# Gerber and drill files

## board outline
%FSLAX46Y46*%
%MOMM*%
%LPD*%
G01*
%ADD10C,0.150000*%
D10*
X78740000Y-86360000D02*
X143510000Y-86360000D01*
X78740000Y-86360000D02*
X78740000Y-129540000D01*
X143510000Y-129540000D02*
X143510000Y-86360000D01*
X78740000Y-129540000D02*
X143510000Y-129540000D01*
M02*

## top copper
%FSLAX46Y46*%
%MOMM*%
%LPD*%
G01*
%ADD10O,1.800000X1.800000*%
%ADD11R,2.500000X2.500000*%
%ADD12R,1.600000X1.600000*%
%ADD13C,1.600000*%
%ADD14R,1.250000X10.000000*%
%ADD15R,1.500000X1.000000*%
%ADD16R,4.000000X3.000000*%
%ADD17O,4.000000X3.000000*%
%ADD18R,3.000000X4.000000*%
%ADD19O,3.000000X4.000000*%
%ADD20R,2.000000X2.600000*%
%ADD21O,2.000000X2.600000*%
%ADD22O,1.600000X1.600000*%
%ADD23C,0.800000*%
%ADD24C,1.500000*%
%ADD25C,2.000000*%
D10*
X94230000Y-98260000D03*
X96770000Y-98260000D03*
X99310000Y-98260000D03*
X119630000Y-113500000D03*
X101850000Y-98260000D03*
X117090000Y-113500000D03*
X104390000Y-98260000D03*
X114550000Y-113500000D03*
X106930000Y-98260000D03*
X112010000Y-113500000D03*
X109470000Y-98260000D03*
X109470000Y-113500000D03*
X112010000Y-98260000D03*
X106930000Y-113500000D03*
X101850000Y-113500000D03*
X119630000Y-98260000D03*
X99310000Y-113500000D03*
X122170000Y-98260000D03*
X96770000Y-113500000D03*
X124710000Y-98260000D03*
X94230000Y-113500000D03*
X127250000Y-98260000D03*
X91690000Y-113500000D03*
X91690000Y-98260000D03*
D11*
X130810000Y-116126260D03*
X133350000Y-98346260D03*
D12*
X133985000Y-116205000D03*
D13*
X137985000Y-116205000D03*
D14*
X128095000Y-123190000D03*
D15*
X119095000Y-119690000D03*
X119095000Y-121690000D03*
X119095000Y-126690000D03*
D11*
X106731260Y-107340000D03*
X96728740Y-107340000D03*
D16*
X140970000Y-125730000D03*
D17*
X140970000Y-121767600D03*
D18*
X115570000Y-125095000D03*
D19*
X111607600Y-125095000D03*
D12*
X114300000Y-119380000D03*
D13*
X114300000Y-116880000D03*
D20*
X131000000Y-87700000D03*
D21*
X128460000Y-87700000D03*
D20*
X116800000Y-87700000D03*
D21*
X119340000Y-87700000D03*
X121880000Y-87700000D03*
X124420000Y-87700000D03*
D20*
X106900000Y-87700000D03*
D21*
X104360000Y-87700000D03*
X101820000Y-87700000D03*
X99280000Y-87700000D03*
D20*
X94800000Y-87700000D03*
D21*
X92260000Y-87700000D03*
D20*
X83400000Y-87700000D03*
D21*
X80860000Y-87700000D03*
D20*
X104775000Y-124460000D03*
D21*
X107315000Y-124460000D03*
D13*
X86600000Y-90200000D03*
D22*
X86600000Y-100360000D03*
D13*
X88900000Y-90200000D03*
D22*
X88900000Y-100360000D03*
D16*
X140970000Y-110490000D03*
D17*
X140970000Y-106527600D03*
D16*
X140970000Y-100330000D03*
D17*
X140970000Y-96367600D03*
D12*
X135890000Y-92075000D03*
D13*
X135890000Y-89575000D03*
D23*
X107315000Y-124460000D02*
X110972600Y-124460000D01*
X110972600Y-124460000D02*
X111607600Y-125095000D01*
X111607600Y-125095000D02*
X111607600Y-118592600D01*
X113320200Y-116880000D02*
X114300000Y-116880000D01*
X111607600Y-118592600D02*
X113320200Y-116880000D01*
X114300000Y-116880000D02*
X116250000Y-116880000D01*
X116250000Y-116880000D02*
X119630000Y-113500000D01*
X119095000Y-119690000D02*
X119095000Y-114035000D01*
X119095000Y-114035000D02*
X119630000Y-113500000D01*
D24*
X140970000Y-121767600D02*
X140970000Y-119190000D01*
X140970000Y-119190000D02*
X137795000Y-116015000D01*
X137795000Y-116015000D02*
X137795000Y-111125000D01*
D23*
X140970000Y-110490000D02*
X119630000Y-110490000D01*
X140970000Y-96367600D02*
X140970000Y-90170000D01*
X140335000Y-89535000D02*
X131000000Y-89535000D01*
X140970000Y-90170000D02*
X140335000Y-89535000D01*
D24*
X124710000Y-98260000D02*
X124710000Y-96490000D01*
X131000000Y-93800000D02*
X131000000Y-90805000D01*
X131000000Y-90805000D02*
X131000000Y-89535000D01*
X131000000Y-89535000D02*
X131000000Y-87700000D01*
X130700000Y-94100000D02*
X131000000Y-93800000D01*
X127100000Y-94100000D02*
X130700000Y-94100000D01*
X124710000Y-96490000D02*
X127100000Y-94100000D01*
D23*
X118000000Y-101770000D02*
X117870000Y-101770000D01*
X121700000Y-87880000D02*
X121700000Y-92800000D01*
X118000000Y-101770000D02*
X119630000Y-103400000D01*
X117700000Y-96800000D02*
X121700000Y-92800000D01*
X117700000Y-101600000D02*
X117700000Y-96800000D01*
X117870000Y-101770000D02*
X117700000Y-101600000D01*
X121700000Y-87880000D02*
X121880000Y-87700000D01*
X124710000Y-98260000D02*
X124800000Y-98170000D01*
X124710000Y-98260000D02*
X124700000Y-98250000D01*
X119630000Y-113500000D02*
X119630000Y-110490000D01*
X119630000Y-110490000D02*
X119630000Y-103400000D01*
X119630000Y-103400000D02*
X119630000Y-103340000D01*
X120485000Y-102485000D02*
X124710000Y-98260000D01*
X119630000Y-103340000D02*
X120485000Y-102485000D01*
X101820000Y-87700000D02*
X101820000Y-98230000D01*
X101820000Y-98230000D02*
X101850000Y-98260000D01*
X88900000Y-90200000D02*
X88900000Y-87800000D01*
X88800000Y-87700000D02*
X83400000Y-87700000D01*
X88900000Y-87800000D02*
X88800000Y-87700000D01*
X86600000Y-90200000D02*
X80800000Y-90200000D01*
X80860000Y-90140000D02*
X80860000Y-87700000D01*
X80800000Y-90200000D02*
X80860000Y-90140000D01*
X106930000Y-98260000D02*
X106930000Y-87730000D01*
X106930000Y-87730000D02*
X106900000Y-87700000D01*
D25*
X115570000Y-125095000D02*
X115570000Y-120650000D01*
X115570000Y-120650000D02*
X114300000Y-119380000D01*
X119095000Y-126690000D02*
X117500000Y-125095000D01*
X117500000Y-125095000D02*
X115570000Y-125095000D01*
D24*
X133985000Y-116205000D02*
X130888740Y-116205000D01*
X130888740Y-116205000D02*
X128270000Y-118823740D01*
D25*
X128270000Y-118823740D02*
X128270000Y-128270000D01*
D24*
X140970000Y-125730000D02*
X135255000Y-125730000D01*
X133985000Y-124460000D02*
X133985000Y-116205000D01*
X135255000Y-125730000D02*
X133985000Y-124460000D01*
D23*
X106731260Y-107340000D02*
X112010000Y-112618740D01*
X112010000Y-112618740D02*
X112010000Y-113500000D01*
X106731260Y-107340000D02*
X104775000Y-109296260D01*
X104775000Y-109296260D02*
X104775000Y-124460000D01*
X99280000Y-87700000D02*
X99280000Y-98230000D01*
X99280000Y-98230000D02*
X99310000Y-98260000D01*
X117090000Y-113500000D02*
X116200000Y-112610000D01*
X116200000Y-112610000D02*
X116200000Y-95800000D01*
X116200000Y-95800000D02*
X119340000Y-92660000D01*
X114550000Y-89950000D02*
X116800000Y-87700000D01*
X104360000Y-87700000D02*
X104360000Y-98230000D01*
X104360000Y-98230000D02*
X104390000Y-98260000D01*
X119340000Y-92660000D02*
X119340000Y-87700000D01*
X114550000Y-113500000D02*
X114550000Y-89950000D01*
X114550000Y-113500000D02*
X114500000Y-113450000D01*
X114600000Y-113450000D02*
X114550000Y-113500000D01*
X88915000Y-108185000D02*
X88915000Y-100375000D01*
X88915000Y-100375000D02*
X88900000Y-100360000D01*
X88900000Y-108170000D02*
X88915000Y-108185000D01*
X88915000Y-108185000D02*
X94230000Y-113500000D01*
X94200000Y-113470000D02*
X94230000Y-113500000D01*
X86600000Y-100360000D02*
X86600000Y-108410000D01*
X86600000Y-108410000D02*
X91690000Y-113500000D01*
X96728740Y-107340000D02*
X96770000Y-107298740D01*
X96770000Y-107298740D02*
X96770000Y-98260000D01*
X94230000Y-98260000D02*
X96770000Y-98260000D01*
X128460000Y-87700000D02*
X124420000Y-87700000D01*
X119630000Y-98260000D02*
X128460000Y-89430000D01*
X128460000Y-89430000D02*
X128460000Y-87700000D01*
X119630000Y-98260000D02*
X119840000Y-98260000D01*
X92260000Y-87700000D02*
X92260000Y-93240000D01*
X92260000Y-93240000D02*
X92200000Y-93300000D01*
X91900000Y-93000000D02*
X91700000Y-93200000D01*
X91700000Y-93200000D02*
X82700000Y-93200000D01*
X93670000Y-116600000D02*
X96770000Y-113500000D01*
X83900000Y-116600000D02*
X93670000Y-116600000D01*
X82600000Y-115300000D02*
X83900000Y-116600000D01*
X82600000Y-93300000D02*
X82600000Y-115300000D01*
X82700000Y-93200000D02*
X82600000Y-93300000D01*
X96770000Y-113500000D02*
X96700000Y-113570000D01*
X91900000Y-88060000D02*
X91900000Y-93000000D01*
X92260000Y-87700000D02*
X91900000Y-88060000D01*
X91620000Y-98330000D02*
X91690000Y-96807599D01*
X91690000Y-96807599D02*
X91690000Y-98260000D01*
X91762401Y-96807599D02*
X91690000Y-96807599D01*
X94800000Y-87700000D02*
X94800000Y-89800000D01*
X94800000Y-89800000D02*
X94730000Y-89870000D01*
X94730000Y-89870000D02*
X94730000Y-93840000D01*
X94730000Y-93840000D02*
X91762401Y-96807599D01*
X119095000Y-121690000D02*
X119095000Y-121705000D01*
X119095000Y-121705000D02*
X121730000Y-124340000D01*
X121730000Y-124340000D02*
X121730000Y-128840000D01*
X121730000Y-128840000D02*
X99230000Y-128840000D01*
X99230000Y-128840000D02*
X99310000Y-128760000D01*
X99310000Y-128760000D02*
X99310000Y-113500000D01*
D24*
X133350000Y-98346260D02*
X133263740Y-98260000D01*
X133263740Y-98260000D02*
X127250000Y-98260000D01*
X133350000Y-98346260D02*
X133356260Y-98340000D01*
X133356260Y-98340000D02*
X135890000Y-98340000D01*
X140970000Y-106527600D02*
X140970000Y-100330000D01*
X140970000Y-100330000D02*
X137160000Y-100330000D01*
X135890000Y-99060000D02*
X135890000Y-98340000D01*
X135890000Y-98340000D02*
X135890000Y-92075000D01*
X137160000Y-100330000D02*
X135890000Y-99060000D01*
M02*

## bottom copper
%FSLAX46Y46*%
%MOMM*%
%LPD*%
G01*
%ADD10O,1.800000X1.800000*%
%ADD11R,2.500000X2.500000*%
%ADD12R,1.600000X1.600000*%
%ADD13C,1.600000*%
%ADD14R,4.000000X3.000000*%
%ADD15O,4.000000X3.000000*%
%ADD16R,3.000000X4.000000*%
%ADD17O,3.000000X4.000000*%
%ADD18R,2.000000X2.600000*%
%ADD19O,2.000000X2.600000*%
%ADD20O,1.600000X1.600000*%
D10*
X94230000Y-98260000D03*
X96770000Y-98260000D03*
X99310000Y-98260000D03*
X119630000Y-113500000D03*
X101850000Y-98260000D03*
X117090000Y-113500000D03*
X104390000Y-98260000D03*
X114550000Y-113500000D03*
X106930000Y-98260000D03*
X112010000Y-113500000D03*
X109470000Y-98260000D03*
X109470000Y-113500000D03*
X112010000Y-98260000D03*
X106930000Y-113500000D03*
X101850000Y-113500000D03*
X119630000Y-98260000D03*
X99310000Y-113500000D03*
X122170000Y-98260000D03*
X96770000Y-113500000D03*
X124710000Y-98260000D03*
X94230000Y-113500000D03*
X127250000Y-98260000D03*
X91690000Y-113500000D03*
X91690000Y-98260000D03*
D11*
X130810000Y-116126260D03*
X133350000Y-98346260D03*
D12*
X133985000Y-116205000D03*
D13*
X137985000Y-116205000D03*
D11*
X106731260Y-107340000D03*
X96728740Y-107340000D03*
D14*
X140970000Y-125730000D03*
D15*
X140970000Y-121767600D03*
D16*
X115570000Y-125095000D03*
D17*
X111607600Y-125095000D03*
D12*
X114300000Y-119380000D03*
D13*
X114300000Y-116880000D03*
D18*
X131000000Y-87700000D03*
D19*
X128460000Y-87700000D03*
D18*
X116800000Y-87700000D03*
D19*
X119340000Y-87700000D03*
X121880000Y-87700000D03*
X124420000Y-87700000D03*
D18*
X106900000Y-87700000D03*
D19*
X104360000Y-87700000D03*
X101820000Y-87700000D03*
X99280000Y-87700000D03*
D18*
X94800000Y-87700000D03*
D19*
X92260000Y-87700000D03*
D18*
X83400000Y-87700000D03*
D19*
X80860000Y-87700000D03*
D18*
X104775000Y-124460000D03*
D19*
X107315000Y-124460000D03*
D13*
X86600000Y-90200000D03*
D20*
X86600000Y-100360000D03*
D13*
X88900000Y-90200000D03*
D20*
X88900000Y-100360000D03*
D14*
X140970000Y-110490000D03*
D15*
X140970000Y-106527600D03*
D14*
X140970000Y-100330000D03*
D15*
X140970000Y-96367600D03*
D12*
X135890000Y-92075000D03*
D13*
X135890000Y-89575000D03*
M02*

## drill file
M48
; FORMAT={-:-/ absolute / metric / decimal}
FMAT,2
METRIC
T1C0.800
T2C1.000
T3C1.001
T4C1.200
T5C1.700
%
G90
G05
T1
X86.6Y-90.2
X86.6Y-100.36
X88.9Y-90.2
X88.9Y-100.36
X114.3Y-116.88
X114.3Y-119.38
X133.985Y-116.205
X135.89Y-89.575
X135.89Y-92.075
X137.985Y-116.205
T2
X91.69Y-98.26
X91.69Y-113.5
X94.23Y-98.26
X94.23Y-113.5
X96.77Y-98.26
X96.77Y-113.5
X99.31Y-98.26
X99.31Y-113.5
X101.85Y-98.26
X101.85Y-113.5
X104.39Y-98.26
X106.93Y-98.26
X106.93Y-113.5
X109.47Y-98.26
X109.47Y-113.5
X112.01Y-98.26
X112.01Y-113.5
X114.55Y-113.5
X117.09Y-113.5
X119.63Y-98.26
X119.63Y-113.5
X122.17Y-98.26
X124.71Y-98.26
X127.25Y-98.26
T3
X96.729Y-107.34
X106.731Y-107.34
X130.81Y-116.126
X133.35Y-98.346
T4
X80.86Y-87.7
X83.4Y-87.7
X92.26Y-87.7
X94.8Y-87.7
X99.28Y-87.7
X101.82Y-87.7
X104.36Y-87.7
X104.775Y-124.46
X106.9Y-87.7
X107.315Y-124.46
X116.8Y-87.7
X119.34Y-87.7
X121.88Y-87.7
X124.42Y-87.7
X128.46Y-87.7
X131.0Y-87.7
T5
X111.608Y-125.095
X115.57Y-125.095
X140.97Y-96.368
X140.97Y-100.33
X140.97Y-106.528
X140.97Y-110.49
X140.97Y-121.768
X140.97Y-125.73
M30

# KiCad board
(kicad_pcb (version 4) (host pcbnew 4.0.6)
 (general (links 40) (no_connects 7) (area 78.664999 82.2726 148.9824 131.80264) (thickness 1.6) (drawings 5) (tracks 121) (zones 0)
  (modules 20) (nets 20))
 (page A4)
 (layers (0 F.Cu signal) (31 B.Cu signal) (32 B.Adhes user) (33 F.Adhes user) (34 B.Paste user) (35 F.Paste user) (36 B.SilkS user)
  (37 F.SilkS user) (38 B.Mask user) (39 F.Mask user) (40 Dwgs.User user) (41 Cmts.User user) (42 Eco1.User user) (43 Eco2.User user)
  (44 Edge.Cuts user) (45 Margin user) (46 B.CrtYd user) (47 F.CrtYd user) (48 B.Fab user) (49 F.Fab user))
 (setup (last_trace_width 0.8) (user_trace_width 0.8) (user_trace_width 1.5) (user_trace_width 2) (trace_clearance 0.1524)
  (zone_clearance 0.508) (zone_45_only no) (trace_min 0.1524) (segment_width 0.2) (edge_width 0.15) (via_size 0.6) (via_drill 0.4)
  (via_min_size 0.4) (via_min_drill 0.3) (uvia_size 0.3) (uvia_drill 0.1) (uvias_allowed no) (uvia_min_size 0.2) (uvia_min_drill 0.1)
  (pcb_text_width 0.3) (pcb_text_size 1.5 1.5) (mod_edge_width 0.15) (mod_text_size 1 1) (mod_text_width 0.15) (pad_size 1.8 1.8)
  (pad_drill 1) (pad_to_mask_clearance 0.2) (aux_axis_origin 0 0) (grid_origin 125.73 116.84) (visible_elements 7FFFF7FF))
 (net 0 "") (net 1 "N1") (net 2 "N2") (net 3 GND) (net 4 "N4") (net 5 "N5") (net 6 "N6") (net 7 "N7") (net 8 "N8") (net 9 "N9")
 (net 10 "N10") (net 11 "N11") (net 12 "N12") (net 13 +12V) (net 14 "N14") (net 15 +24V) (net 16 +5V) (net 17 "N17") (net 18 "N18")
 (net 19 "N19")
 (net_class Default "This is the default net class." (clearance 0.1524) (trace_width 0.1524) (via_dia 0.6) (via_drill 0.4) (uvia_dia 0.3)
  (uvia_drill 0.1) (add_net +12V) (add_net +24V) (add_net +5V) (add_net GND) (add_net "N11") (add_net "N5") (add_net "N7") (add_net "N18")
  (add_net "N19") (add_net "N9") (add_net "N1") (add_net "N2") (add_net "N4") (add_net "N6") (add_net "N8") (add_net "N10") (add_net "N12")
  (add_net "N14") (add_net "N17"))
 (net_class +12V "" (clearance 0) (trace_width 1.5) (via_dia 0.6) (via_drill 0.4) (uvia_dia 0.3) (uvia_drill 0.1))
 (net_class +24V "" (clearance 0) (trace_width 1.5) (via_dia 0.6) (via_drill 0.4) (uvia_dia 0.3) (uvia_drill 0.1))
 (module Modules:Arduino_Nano (layer B.Cu) (at 127.25 113.5 90)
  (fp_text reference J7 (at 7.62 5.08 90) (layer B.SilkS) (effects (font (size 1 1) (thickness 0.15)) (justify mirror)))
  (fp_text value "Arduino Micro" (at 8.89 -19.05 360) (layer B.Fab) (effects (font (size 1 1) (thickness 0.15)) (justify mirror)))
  (pad 3.3V thru_hole oval (at 15.24 -33.02 90) (size 1.8 1.8) (drill 1) (layers *.Cu *.Mask) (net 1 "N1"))
  (pad AREF thru_hole oval (at 15.24 -30.48 90) (size 1.8 1.8) (drill 1) (layers *.Cu *.Mask) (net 1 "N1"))
  (pad A0 thru_hole oval (at 15.24 -27.94 90) (size 1.8 1.8) (drill 1) (layers *.Cu *.Mask) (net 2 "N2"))
  (pad GND thru_hole oval (at 0 -7.62 90) (size 1.8 1.8) (drill 1) (layers *.Cu *.Mask) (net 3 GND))
  (pad A1 thru_hole oval (at 15.24 -25.4 90) (size 1.8 1.8) (drill 1) (layers *.Cu *.Mask) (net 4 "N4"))
  (pad SDA thru_hole oval (at 0 -10.16 90) (size 1.8 1.8) (drill 1) (layers *.Cu *.Mask) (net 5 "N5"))
  (pad A2 thru_hole oval (at 15.24 -22.86 90) (size 1.8 1.8) (drill 1) (layers *.Cu *.Mask) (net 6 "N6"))
  (pad SCL thru_hole oval (at 0 -12.7 90) (size 1.8 1.8) (drill 1) (layers *.Cu *.Mask) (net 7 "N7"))
  (pad A3 thru_hole oval (at 15.24 -20.32 90) (size 1.8 1.8) (drill 1) (layers *.Cu *.Mask) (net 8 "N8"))
  (pad D4 thru_hole oval (at 0 -15.24 90) (size 1.8 1.8) (drill 1) (layers *.Cu *.Mask) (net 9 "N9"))
  (pad A4 thru_hole oval (at 15.24 -17.78 90) (size 1.8 1.8) (drill 1) (layers *.Cu *.Mask) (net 9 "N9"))
  (pad D5 thru_hole oval (at 0 -17.78 90) (size 1.8 1.8) (drill 1) (layers *.Cu *.Mask))
  (pad A5 thru_hole oval (at 15.24 -15.24 90) (size 1.8 1.8) (drill 1) (layers *.Cu *.Mask) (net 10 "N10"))
  (pad D6 thru_hole oval (at 0 -20.32 90) (size 1.8 1.8) (drill 1) (layers *.Cu *.Mask))
  (pad D8 thru_hole oval (at 0 -25.4 90) (size 1.8 1.8) (drill 1) (layers *.Cu *.Mask))
  (pad 5v thru_hole oval (at 15.24 -7.62 90) (size 1.8 1.8) (drill 1) (layers *.Cu *.Mask))
  (pad D9 thru_hole oval (at 0 -27.94 90) (size 1.8 1.8) (drill 1) (layers *.Cu *.Mask) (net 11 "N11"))
  (pad RS thru_hole oval (at 15.24 -5.08 90) (size 1.8 1.8) (drill 1) (layers *.Cu *.Mask))
  (pad D10 thru_hole oval (at 0 -30.48 90) (size 1.8 1.8) (drill 1) (layers *.Cu *.Mask))
  (pad GND thru_hole oval (at 15.24 -2.54 90) (size 1.8 1.8) (drill 1) (layers *.Cu *.Mask) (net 3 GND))
  (pad D11 thru_hole oval (at 0 -33.02 90) (size 1.8 1.8) (drill 1) (layers *.Cu *.Mask) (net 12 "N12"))
  (pad Vin thru_hole oval (at 15.24 0 90) (size 1.8 1.8) (drill 1) (layers *.Cu *.Mask) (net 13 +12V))
  (pad D12 thru_hole oval (at 0 -35.56 90) (size 1.8 1.8) (drill 1) (layers *.Cu *.Mask) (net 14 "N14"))
  (pad D13 thru_hole oval (at 15.24 -35.56 90) (size 1.8 1.8) (drill 1) (layers *.Cu *.Mask)))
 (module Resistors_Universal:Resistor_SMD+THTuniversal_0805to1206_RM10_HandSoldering (layer F.Cu) (at 130.81 111.125 90)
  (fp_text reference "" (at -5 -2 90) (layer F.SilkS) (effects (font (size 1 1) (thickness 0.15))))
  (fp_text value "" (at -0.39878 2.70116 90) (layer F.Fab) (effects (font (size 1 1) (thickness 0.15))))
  (pad 1 thru_hole rect (at -5.00126 0 270) (size 2.5 2.5) (drill 1.00076) (layers *.Cu *.Mask) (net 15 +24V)))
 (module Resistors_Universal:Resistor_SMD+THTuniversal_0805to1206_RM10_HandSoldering (layer F.Cu) (at 133.35 93.345 90)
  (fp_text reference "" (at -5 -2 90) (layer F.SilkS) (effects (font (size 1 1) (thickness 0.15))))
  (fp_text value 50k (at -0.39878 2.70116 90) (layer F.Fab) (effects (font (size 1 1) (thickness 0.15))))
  (pad 1 thru_hole rect (at -5.00126 0 270) (size 2.5 2.5) (drill 1.00076) (layers *.Cu *.Mask) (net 13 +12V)))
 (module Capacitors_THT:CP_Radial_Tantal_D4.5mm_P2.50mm (layer B.Cu) (at 133.985 116.205)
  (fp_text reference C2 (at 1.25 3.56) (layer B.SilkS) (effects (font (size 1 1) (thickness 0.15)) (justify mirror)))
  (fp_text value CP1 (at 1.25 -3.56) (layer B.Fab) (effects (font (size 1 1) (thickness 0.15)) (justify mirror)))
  (pad 1 thru_hole rect (at 0 0) (size 1.6 1.6) (drill 0.8) (layers *.Cu *.Mask) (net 15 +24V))
  (pad 2 thru_hole circle (at 4 0) (size 1.6 1.6) (drill 0.8) (layers *.Cu *.Mask) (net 3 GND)))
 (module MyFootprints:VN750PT (layer F.Cu) (at 125.095 123.19 270)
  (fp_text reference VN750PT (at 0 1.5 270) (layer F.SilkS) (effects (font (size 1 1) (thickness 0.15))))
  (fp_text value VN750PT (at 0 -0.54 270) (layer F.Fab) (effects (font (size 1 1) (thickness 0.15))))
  (pad Vcc smd rect (at 0 -3 270) (size 10 1.25) (layers F.Cu F.Paste F.Mask) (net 15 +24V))
  (pad GND smd rect (at -3.5 6 270) (size 1 1.5) (layers F.Cu F.Paste F.Mask) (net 3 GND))
  (pad Inpu smd rect (at -1.5 6 270) (size 1 1.5) (layers F.Cu F.Paste F.Mask) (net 11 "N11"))
  (pad Vout smd rect (at 3.5 6 270) (size 1 1.5) (layers F.Cu F.Paste F.Mask) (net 15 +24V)))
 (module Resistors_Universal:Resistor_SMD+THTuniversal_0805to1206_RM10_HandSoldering (layer F.Cu) (at 101.73 107.34 180)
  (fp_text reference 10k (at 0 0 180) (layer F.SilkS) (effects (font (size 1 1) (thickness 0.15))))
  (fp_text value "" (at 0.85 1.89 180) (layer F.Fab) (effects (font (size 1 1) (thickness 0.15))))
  (pad 1 thru_hole rect (at -5.00126 0) (size 2.5 2.5) (drill 1.00076) (layers *.Cu *.Mask) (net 9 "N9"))
  (pad 2 thru_hole rect (at 5.00126 0) (size 2.5 2.5) (drill 1.00076) (layers *.Cu *.Mask) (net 1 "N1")))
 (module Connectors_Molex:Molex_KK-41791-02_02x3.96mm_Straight (layer F.Cu) (at 140.97 125.73 90)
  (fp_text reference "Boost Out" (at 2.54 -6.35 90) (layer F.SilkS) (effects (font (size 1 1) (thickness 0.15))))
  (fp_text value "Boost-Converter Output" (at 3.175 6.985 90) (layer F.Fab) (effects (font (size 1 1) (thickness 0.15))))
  (pad 1 thru_hole rect (at 0 0 90) (size 3 4) (drill 1.7) (layers *.Cu *.Mask) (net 15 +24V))
  (pad 2 thru_hole oval (at 3.9624 0 90) (size 3 4) (drill 1.7) (layers *.Cu *.Mask) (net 3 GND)))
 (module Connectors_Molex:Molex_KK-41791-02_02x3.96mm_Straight (layer F.Cu) (at 115.57 125.095 180)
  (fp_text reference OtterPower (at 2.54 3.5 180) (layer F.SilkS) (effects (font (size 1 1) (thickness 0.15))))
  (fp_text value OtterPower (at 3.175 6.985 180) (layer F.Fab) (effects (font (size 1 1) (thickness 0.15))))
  (pad 1 thru_hole rect (at 0 0 180) (size 3 4) (drill 1.7) (layers *.Cu *.Mask) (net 15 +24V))
  (pad 2 thru_hole oval (at 3.9624 0 180) (size 3 4) (drill 1.7) (layers *.Cu *.Mask) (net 3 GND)))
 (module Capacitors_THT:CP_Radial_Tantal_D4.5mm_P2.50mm (layer B.Cu) (at 114.3 119.38 90)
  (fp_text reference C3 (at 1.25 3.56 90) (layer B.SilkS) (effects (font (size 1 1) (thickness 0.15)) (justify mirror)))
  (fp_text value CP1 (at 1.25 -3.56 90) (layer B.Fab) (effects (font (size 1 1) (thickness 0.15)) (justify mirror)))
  (pad + thru_hole rect (at 0 0 90) (size 1.6 1.6) (drill 0.8) (layers *.Cu *.Mask) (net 15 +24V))
  (pad 2 thru_hole circle (at 2.5 0 90) (size 1.6 1.6) (drill 0.8) (layers *.Cu *.Mask) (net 3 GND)))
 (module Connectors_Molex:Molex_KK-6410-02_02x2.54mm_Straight (layer F.Cu) (at 131 87.7 180)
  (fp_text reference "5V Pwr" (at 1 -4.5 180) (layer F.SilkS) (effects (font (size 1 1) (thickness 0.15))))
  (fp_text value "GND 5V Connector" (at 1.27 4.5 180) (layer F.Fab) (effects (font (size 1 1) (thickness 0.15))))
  (pad 1 thru_hole rect (at 0 0 180) (size 2 2.6) (drill 1.2) (layers *.Cu *.Mask) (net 3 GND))
  (pad 2 thru_hole oval (at 2.54 0 180) (size 2 2.6) (drill 1.2) (layers *.Cu *.Mask) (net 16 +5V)))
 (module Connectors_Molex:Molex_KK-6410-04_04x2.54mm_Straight (layer F.Cu) (at 116.8 87.7)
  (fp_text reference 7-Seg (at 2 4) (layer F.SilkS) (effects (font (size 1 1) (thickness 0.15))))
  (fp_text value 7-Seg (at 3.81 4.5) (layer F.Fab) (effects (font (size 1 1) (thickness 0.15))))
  (pad 1 thru_hole rect (at 0 0) (size 2 2.6) (drill 1.2) (layers *.Cu *.Mask) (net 5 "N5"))
  (pad 2 thru_hole oval (at 2.54 0) (size 2 2.6) (drill 1.2) (layers *.Cu *.Mask) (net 7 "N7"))
  (pad 3 thru_hole oval (at 5.08 0) (size 2 2.6) (drill 1.2) (layers *.Cu *.Mask) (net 3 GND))
  (pad 4 thru_hole oval (at 7.62 0) (size 2 2.6) (drill 1.2) (layers *.Cu *.Mask) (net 16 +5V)))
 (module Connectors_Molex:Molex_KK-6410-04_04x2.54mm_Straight (layer F.Cu) (at 106.9 87.7 180)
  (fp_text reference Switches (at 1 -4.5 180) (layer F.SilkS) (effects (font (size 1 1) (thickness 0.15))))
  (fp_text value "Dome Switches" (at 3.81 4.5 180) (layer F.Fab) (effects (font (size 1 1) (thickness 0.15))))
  (pad 1 thru_hole rect (at 0 0 180) (size 2 2.6) (drill 1.2) (layers *.Cu *.Mask) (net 8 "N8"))
  (pad 2 thru_hole oval (at 2.54 0 180) (size 2 2.6) (drill 1.2) (layers *.Cu *.Mask) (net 6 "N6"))
  (pad 3 thru_hole oval (at 5.08 0 180) (size 2 2.6) (drill 1.2) (layers *.Cu *.Mask) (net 4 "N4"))
  (pad 4 thru_hole oval (at 7.62 0 180) (size 2 2.6) (drill 1.2) (layers *.Cu *.Mask) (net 2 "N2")))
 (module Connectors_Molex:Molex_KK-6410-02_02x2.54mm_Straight (layer F.Cu) (at 94.8 87.7 180)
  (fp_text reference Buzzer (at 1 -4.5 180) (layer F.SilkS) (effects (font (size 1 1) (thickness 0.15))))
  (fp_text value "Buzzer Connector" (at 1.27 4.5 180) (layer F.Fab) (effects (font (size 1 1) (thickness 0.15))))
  (pad 1 thru_hole rect (at 0 0 180) (size 2 2.6) (drill 1.2) (layers *.Cu *.Mask) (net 10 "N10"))
  (pad 2 thru_hole oval (at 2.54 0 180) (size 2 2.6) (drill 1.2) (layers *.Cu *.Mask) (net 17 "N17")))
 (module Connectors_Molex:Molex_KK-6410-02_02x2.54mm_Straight (layer F.Cu) (at 83.4 87.7 180)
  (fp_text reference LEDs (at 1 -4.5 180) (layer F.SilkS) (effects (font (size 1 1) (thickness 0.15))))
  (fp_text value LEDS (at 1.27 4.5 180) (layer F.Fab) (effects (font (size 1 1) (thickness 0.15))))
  (pad 1 thru_hole rect (at 0 0 180) (size 2 2.6) (drill 1.2) (layers *.Cu *.Mask) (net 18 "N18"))
  (pad 2 thru_hole oval (at 2.54 0 180) (size 2 2.6) (drill 1.2) (layers *.Cu *.Mask) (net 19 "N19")))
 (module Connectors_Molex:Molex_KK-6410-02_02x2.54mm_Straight (layer F.Cu) (at 104.775 124.46)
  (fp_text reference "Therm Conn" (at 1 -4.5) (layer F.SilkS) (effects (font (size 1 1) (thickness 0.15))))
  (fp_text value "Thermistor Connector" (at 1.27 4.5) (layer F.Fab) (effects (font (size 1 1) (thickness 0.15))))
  (pad 1 thru_hole rect (at 0 0) (size 2 2.6) (drill 1.2) (layers *.Cu *.Mask) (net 9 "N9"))
  (pad 2 thru_hole oval (at 2.54 0) (size 2 2.6) (drill 1.2) (layers *.Cu *.Mask) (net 3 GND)))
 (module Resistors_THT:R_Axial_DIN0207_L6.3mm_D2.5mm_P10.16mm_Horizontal (layer F.Cu) (at 86.6 90.2 270)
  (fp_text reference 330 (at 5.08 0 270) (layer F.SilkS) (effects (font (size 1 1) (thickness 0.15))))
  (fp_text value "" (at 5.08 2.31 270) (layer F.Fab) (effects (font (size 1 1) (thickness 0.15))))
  (pad 1 thru_hole circle (at 0 0 270) (size 1.6 1.6) (drill 0.8) (layers *.Cu *.Mask) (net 19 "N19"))
  (pad 2 thru_hole oval (at 10.16 0 270) (size 1.6 1.6) (drill 0.8) (layers *.Cu *.Mask) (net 14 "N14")))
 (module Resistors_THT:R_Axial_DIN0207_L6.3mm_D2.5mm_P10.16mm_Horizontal (layer F.Cu) (at 88.9 90.2 270)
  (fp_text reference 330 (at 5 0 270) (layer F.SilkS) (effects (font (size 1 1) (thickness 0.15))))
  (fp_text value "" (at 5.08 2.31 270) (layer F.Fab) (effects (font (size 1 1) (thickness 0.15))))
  (pad 1 thru_hole circle (at 0 0 270) (size 1.6 1.6) (drill 0.8) (layers *.Cu *.Mask) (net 18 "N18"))
  (pad 2 thru_hole oval (at 10.16 0 270) (size 1.6 1.6) (drill 0.8) (layers *.Cu *.Mask) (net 12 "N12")))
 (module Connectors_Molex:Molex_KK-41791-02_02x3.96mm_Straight (layer F.Cu) (at 140.97 110.49 90)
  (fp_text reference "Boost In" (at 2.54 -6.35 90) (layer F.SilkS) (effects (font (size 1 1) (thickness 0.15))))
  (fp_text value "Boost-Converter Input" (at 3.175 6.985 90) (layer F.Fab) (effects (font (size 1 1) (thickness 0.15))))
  (pad 1 thru_hole rect (at 0 0 90) (size 3 4) (drill 1.7) (layers *.Cu *.Mask) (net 3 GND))
  (pad 2 thru_hole oval (at 3.9624 0 90) (size 3 4) (drill 1.7) (layers *.Cu *.Mask) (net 13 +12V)))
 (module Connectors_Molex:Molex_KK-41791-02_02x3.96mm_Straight (layer F.Cu) (at 140.97 100.33 90)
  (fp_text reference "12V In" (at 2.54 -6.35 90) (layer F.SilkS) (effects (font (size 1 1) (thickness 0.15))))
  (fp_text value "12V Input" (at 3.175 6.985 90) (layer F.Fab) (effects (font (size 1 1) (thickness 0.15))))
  (pad 1 thru_hole rect (at 0 0 90) (size 3 4) (drill 1.7) (layers *.Cu *.Mask) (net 13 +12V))
  (pad 2 thru_hole oval (at 3.9624 0 90) (size 3 4) (drill 1.7) (layers *.Cu *.Mask) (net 3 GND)))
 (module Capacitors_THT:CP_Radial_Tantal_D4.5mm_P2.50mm (layer F.Cu) (at 135.89 92.075 90)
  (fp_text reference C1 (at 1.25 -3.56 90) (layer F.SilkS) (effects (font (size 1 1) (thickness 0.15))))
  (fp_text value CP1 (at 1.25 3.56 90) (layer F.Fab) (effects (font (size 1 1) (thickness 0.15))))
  (pad 1 thru_hole rect (at 0 0 90) (size 1.6 1.6) (drill 0.8) (layers *.Cu *.Mask) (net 13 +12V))
  (pad 2 thru_hole circle (at 2.5 0 90) (size 1.6 1.6) (drill 0.8) (layers *.Cu *.Mask) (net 3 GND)))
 (gr_line (start 78.74 86.36) (end 143.51 86.36) (angle 90) (layer Edge.Cuts) (width 0.15))
 (gr_line (start 78.74 86.36) (end 78.74 129.54) (angle 90) (layer Edge.Cuts) (width 0.15))
 (gr_line (start 143.51 129.54) (end 143.51 86.36) (angle 90) (layer Edge.Cuts) (width 0.15))
 (gr_line (start 78.74 129.54) (end 143.51 129.54) (angle 90) (layer Edge.Cuts) (width 0.15))
 (segment (start 107.315 124.46) (end 110.9726 124.46) (width 0.8) (layer F.Cu) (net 3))
 (segment (start 110.9726 124.46) (end 111.6076 125.095) (width 0.8) (layer F.Cu) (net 3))
 (segment (start 111.6076 125.095) (end 111.6076 118.5926) (width 0.8) (layer F.Cu) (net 3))
 (segment (start 113.3202 116.88) (end 114.3 116.88) (width 0.8) (layer F.Cu) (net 3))
 (segment (start 111.6076 118.5926) (end 113.3202 116.88) (width 0.8) (layer F.Cu) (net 3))
 (segment (start 114.3 116.88) (end 116.25 116.88) (width 0.8) (layer F.Cu) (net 3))
 (segment (start 116.25 116.88) (end 119.63 113.5) (width 0.8) (layer F.Cu) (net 3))
 (segment (start 119.095 119.69) (end 119.095 114.035) (width 0.8) (layer F.Cu) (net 3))
 (segment (start 119.095 114.035) (end 119.63 113.5) (width 0.8) (layer F.Cu) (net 3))
 (segment (start 140.97 121.7676) (end 140.97 119.19) (width 1.5) (layer F.Cu) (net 3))
 (segment (start 140.97 119.19) (end 137.795 116.015) (width 1.5) (layer F.Cu) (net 3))
 (segment (start 137.795 116.015) (end 137.795 111.125) (width 1.5) (layer F.Cu) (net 3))
 (segment (start 140.97 110.49) (end 119.63 110.49) (width 0.8) (layer F.Cu) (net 3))
 (segment (start 140.97 96.3676) (end 140.97 90.17) (width 0.8) (layer F.Cu) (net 3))
 (segment (start 140.335 89.535) (end 131 89.535) (width 0.8) (layer F.Cu) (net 3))
 (segment (start 140.97 90.17) (end 140.335 89.535) (width 0.8) (layer F.Cu) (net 3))
 (segment (start 124.71 98.26) (end 124.71 96.49) (width 1.5) (layer F.Cu) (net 3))
 (segment (start 131 93.8) (end 131 90.805) (width 1.5) (layer F.Cu) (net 3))
 (segment (start 131 90.805) (end 131 89.535) (width 1.5) (layer F.Cu) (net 3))
 (segment (start 131 89.535) (end 131 87.7) (width 1.5) (layer F.Cu) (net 3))
 (segment (start 130.7 94.1) (end 131 93.8) (width 1.5) (layer F.Cu) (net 3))
 (segment (start 127.1 94.1) (end 130.7 94.1) (width 1.5) (layer F.Cu) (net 3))
 (segment (start 124.71 96.49) (end 127.1 94.1) (width 1.5) (layer F.Cu) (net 3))
 (segment (start 118 101.77) (end 117.87 101.77) (width 0.8) (layer F.Cu) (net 3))
 (segment (start 121.7 87.88) (end 121.7 92.8) (width 0.8) (layer F.Cu) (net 3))
 (segment (start 118 101.77) (end 119.63 103.4) (width 0.8) (layer F.Cu) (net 3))
 (segment (start 117.7 96.8) (end 121.7 92.8) (width 0.8) (layer F.Cu) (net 3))
 (segment (start 117.7 101.6) (end 117.7 96.8) (width 0.8) (layer F.Cu) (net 3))
 (segment (start 117.87 101.77) (end 117.7 101.6) (width 0.8) (layer F.Cu) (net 3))
 (segment (start 121.7 87.88) (end 121.88 87.7) (width 0.8) (layer F.Cu) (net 3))
 (segment (start 124.71 98.26) (end 124.8 98.17) (width 0.8) (layer F.Cu) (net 3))
 (segment (start 124.71 98.26) (end 124.7 98.25) (width 0.8) (layer F.Cu) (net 3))
 (segment (start 119.63 113.5) (end 119.63 110.49) (width 0.8) (layer F.Cu) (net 3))
 (segment (start 119.63 110.49) (end 119.63 103.4) (width 0.8) (layer F.Cu) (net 3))
 (segment (start 119.63 103.4) (end 119.63 103.34) (width 0.8) (layer F.Cu) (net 3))
 (segment (start 120.485 102.485) (end 124.71 98.26) (width 0.8) (layer F.Cu) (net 3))
 (segment (start 119.63 103.34) (end 120.485 102.485) (width 0.8) (layer F.Cu) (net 3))
 (segment (start 101.82 87.7) (end 101.82 98.23) (width 0.8) (layer F.Cu) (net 4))
 (segment (start 101.82 98.23) (end 101.85 98.26) (width 0.8) (layer F.Cu) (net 4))
 (segment (start 88.9 90.2) (end 88.9 87.8) (width 0.8) (layer F.Cu) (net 18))
 (segment (start 88.8 87.7) (end 83.4 87.7) (width 0.8) (layer F.Cu) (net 18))
 (segment (start 88.9 87.8) (end 88.8 87.7) (width 0.8) (layer F.Cu) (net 18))
 (segment (start 86.6 90.2) (end 80.8 90.2) (width 0.8) (layer F.Cu) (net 19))
 (segment (start 80.86 90.14) (end 80.86 87.7) (width 0.8) (layer F.Cu) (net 19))
 (segment (start 80.8 90.2) (end 80.86 90.14) (width 0.8) (layer F.Cu) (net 19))
 (segment (start 106.93 98.26) (end 106.93 87.73) (width 0.8) (layer F.Cu) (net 8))
 (segment (start 106.93 87.73) (end 106.9 87.7) (width 0.8) (layer F.Cu) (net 8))
 (segment (start 115.57 125.095) (end 115.57 120.65) (width 2) (layer F.Cu) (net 15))
 (segment (start 115.57 120.65) (end 114.3 119.38) (width 2) (layer F.Cu) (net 15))
 (segment (start 119.095 126.69) (end 117.5 125.095) (width 2) (layer F.Cu) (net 15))
 (segment (start 117.5 125.095) (end 115.57 125.095) (width 2) (layer F.Cu) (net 15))
 (segment (start 133.985 116.205) (end 130.88874 116.205) (width 1.5) (layer F.Cu) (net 15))
 (segment (start 130.88874 116.205) (end 128.27 118.82374) (width 1.5) (layer F.Cu) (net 15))
 (segment (start 128.27 118.82374) (end 128.27 128.27) (width 2) (layer F.Cu) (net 15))
 (segment (start 140.97 125.73) (end 135.255 125.73) (width 1.5) (layer F.Cu) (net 15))
 (segment (start 133.985 124.46) (end 133.985 116.205) (width 1.5) (layer F.Cu) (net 15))
 (segment (start 135.255 125.73) (end 133.985 124.46) (width 1.5) (layer F.Cu) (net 15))
 (segment (start 106.73126 107.34) (end 112.01 112.61874) (width 0.8) (layer F.Cu) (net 9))
 (segment (start 112.01 112.61874) (end 112.01 113.5) (width 0.8) (layer F.Cu) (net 9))
 (segment (start 106.73126 107.34) (end 104.775 109.29626) (width 0.8) (layer F.Cu) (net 9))
 (segment (start 104.775 109.29626) (end 104.775 124.46) (width 0.8) (layer F.Cu) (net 9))
 (segment (start 99.28 87.7) (end 99.28 98.23) (width 0.8) (layer F.Cu) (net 2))
 (segment (start 99.28 98.23) (end 99.31 98.26) (width 0.8) (layer F.Cu) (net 2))
 (segment (start 117.09 113.5) (end 116.2 112.61) (width 0.8) (layer F.Cu) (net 5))
 (segment (start 116.2 112.61) (end 116.2 95.8) (width 0.8) (layer F.Cu) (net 5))
 (segment (start 116.2 95.8) (end 119.34 92.66) (width 0.8) (layer F.Cu) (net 5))
 (segment (start 114.55 89.95) (end 116.8 87.7) (width 0.8) (layer F.Cu) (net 5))
 (segment (start 104.36 87.7) (end 104.36 98.23) (width 0.8) (layer F.Cu) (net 6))
 (segment (start 104.36 98.23) (end 104.39 98.26) (width 0.8) (layer F.Cu) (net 6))
 (segment (start 119.34 92.66) (end 119.34 87.7) (width 0.8) (layer F.Cu) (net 7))
 (segment (start 114.55 113.5) (end 114.55 89.95) (width 0.8) (layer F.Cu) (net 7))
 (segment (start 114.55 113.5) (end 114.5 113.45) (width 0.8) (layer F.Cu) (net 7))
 (segment (start 114.6 113.45) (end 114.55 113.5) (width 0.8) (layer F.Cu) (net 7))
 (segment (start 88.915 108.185) (end 88.915 100.375) (width 0.8) (layer F.Cu) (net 12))
 (segment (start 88.915 100.375) (end 88.9 100.36) (width 0.8) (layer F.Cu) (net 12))
 (segment (start 88.9 108.17) (end 88.915 108.185) (width 0.8) (layer F.Cu) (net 12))
 (segment (start 88.915 108.185) (end 94.23 113.5) (width 0.8) (layer F.Cu) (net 12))
 (segment (start 94.2 113.47) (end 94.23 113.5) (width 0.8) (layer F.Cu) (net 12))
 (segment (start 86.6 100.36) (end 86.6 108.41) (width 0.8) (layer F.Cu) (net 14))
 (segment (start 86.6 108.41) (end 91.69 113.5) (width 0.8) (layer F.Cu) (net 14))
 (segment (start 96.72874 107.34) (end 96.77 107.29874) (width 0.8) (layer F.Cu) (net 1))
 (segment (start 96.77 107.29874) (end 96.77 98.26) (width 0.8) (layer F.Cu) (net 1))
 (segment (start 94.23 98.26) (end 96.77 98.26) (width 0.8) (layer F.Cu) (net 1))
 (segment (start 128.46 87.7) (end 124.42 87.7) (width 0.8) (layer F.Cu) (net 16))
 (segment (start 119.63 98.26) (end 128.46 89.43) (width 0.8) (layer F.Cu) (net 16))
 (segment (start 128.46 89.43) (end 128.46 87.7) (width 0.8) (layer F.Cu) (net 16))
 (segment (start 119.63 98.26) (end 119.84 98.26) (width 0.8) (layer F.Cu) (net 16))
 (segment (start 92.26 87.7) (end 92.26 93.24) (width 0.8) (layer F.Cu) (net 17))
 (segment (start 92.26 93.24) (end 92.2 93.3) (width 0.8) (layer F.Cu) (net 17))
 (segment (start 91.9 93) (end 91.7 93.2) (width 0.8) (layer F.Cu) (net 17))
 (segment (start 91.7 93.2) (end 82.7 93.2) (width 0.8) (layer F.Cu) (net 17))
 (segment (start 93.67 116.6) (end 96.77 113.5) (width 0.8) (layer F.Cu) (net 17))
 (segment (start 83.9 116.6) (end 93.67 116.6) (width 0.8) (layer F.Cu) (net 17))
 (segment (start 82.6 115.3) (end 83.9 116.6) (width 0.8) (layer F.Cu) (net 17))
 (segment (start 82.6 93.3) (end 82.6 115.3) (width 0.8) (layer F.Cu) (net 17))
 (segment (start 82.7 93.2) (end 82.6 93.3) (width 0.8) (layer F.Cu) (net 17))
 (segment (start 96.77 113.5) (end 96.7 113.57) (width 0.8) (layer F.Cu) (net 17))
 (segment (start 91.9 88.06) (end 91.9 93) (width 0.8) (layer F.Cu) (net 17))
 (segment (start 92.26 87.7) (end 91.9 88.06) (width 0.8) (layer F.Cu) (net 17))
 (segment (start 91.62 98.33) (end 91.69 96.807599) (width 0.8) (layer F.Cu) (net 10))
 (segment (start 91.69 96.807599) (end 91.69 98.26) (width 0.8) (layer F.Cu) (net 10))
 (segment (start 91.762401 96.807599) (end 91.69 96.807599) (width 0.8) (layer F.Cu) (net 10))
 (segment (start 94.8 87.7) (end 94.8 89.8) (width 0.8) (layer F.Cu) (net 10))
 (segment (start 94.8 89.8) (end 94.73 89.87) (width 0.8) (layer F.Cu) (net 10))
 (segment (start 94.73 89.87) (end 94.73 93.84) (width 0.8) (layer F.Cu) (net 10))
 (segment (start 94.73 93.84) (end 91.762401 96.807599) (width 0.8) (layer F.Cu) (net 10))
 (segment (start 119.095 121.69) (end 119.095 121.705) (width 0.8) (layer F.Cu) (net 11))
 (segment (start 119.095 121.705) (end 121.73 124.34) (width 0.8) (layer F.Cu) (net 11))
 (segment (start 121.73 124.34) (end 121.73 128.84) (width 0.8) (layer F.Cu) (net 11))
 (segment (start 121.73 128.84) (end 99.23 128.84) (width 0.8) (layer F.Cu) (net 11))
 (segment (start 99.23 128.84) (end 99.31 128.76) (width 0.8) (layer F.Cu) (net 11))
 (segment (start 99.31 128.76) (end 99.31 113.5) (width 0.8) (layer F.Cu) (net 11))
 (segment (start 133.35 98.34626) (end 133.26374 98.26) (width 1.5) (layer F.Cu) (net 13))
 (segment (start 133.26374 98.26) (end 127.25 98.26) (width 1.5) (layer F.Cu) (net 13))
 (segment (start 133.35 98.34626) (end 133.35626 98.34) (width 1.5) (layer F.Cu) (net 13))
 (segment (start 133.35626 98.34) (end 135.89 98.34) (width 1.5) (layer F.Cu) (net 13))
 (segment (start 140.97 106.5276) (end 140.97 100.33) (width 1.5) (layer F.Cu) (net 13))
 (segment (start 140.97 100.33) (end 137.16 100.33) (width 1.5) (layer F.Cu) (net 13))
 (segment (start 135.89 99.06) (end 135.89 98.34) (width 1.5) (layer F.Cu) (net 13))
 (segment (start 135.89 98.34) (end 135.89 92.075) (width 1.5) (layer F.Cu) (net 13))
 (segment (start 137.16 100.33) (end 135.89 99.06) (width 1.5) (layer F.Cu) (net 13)))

